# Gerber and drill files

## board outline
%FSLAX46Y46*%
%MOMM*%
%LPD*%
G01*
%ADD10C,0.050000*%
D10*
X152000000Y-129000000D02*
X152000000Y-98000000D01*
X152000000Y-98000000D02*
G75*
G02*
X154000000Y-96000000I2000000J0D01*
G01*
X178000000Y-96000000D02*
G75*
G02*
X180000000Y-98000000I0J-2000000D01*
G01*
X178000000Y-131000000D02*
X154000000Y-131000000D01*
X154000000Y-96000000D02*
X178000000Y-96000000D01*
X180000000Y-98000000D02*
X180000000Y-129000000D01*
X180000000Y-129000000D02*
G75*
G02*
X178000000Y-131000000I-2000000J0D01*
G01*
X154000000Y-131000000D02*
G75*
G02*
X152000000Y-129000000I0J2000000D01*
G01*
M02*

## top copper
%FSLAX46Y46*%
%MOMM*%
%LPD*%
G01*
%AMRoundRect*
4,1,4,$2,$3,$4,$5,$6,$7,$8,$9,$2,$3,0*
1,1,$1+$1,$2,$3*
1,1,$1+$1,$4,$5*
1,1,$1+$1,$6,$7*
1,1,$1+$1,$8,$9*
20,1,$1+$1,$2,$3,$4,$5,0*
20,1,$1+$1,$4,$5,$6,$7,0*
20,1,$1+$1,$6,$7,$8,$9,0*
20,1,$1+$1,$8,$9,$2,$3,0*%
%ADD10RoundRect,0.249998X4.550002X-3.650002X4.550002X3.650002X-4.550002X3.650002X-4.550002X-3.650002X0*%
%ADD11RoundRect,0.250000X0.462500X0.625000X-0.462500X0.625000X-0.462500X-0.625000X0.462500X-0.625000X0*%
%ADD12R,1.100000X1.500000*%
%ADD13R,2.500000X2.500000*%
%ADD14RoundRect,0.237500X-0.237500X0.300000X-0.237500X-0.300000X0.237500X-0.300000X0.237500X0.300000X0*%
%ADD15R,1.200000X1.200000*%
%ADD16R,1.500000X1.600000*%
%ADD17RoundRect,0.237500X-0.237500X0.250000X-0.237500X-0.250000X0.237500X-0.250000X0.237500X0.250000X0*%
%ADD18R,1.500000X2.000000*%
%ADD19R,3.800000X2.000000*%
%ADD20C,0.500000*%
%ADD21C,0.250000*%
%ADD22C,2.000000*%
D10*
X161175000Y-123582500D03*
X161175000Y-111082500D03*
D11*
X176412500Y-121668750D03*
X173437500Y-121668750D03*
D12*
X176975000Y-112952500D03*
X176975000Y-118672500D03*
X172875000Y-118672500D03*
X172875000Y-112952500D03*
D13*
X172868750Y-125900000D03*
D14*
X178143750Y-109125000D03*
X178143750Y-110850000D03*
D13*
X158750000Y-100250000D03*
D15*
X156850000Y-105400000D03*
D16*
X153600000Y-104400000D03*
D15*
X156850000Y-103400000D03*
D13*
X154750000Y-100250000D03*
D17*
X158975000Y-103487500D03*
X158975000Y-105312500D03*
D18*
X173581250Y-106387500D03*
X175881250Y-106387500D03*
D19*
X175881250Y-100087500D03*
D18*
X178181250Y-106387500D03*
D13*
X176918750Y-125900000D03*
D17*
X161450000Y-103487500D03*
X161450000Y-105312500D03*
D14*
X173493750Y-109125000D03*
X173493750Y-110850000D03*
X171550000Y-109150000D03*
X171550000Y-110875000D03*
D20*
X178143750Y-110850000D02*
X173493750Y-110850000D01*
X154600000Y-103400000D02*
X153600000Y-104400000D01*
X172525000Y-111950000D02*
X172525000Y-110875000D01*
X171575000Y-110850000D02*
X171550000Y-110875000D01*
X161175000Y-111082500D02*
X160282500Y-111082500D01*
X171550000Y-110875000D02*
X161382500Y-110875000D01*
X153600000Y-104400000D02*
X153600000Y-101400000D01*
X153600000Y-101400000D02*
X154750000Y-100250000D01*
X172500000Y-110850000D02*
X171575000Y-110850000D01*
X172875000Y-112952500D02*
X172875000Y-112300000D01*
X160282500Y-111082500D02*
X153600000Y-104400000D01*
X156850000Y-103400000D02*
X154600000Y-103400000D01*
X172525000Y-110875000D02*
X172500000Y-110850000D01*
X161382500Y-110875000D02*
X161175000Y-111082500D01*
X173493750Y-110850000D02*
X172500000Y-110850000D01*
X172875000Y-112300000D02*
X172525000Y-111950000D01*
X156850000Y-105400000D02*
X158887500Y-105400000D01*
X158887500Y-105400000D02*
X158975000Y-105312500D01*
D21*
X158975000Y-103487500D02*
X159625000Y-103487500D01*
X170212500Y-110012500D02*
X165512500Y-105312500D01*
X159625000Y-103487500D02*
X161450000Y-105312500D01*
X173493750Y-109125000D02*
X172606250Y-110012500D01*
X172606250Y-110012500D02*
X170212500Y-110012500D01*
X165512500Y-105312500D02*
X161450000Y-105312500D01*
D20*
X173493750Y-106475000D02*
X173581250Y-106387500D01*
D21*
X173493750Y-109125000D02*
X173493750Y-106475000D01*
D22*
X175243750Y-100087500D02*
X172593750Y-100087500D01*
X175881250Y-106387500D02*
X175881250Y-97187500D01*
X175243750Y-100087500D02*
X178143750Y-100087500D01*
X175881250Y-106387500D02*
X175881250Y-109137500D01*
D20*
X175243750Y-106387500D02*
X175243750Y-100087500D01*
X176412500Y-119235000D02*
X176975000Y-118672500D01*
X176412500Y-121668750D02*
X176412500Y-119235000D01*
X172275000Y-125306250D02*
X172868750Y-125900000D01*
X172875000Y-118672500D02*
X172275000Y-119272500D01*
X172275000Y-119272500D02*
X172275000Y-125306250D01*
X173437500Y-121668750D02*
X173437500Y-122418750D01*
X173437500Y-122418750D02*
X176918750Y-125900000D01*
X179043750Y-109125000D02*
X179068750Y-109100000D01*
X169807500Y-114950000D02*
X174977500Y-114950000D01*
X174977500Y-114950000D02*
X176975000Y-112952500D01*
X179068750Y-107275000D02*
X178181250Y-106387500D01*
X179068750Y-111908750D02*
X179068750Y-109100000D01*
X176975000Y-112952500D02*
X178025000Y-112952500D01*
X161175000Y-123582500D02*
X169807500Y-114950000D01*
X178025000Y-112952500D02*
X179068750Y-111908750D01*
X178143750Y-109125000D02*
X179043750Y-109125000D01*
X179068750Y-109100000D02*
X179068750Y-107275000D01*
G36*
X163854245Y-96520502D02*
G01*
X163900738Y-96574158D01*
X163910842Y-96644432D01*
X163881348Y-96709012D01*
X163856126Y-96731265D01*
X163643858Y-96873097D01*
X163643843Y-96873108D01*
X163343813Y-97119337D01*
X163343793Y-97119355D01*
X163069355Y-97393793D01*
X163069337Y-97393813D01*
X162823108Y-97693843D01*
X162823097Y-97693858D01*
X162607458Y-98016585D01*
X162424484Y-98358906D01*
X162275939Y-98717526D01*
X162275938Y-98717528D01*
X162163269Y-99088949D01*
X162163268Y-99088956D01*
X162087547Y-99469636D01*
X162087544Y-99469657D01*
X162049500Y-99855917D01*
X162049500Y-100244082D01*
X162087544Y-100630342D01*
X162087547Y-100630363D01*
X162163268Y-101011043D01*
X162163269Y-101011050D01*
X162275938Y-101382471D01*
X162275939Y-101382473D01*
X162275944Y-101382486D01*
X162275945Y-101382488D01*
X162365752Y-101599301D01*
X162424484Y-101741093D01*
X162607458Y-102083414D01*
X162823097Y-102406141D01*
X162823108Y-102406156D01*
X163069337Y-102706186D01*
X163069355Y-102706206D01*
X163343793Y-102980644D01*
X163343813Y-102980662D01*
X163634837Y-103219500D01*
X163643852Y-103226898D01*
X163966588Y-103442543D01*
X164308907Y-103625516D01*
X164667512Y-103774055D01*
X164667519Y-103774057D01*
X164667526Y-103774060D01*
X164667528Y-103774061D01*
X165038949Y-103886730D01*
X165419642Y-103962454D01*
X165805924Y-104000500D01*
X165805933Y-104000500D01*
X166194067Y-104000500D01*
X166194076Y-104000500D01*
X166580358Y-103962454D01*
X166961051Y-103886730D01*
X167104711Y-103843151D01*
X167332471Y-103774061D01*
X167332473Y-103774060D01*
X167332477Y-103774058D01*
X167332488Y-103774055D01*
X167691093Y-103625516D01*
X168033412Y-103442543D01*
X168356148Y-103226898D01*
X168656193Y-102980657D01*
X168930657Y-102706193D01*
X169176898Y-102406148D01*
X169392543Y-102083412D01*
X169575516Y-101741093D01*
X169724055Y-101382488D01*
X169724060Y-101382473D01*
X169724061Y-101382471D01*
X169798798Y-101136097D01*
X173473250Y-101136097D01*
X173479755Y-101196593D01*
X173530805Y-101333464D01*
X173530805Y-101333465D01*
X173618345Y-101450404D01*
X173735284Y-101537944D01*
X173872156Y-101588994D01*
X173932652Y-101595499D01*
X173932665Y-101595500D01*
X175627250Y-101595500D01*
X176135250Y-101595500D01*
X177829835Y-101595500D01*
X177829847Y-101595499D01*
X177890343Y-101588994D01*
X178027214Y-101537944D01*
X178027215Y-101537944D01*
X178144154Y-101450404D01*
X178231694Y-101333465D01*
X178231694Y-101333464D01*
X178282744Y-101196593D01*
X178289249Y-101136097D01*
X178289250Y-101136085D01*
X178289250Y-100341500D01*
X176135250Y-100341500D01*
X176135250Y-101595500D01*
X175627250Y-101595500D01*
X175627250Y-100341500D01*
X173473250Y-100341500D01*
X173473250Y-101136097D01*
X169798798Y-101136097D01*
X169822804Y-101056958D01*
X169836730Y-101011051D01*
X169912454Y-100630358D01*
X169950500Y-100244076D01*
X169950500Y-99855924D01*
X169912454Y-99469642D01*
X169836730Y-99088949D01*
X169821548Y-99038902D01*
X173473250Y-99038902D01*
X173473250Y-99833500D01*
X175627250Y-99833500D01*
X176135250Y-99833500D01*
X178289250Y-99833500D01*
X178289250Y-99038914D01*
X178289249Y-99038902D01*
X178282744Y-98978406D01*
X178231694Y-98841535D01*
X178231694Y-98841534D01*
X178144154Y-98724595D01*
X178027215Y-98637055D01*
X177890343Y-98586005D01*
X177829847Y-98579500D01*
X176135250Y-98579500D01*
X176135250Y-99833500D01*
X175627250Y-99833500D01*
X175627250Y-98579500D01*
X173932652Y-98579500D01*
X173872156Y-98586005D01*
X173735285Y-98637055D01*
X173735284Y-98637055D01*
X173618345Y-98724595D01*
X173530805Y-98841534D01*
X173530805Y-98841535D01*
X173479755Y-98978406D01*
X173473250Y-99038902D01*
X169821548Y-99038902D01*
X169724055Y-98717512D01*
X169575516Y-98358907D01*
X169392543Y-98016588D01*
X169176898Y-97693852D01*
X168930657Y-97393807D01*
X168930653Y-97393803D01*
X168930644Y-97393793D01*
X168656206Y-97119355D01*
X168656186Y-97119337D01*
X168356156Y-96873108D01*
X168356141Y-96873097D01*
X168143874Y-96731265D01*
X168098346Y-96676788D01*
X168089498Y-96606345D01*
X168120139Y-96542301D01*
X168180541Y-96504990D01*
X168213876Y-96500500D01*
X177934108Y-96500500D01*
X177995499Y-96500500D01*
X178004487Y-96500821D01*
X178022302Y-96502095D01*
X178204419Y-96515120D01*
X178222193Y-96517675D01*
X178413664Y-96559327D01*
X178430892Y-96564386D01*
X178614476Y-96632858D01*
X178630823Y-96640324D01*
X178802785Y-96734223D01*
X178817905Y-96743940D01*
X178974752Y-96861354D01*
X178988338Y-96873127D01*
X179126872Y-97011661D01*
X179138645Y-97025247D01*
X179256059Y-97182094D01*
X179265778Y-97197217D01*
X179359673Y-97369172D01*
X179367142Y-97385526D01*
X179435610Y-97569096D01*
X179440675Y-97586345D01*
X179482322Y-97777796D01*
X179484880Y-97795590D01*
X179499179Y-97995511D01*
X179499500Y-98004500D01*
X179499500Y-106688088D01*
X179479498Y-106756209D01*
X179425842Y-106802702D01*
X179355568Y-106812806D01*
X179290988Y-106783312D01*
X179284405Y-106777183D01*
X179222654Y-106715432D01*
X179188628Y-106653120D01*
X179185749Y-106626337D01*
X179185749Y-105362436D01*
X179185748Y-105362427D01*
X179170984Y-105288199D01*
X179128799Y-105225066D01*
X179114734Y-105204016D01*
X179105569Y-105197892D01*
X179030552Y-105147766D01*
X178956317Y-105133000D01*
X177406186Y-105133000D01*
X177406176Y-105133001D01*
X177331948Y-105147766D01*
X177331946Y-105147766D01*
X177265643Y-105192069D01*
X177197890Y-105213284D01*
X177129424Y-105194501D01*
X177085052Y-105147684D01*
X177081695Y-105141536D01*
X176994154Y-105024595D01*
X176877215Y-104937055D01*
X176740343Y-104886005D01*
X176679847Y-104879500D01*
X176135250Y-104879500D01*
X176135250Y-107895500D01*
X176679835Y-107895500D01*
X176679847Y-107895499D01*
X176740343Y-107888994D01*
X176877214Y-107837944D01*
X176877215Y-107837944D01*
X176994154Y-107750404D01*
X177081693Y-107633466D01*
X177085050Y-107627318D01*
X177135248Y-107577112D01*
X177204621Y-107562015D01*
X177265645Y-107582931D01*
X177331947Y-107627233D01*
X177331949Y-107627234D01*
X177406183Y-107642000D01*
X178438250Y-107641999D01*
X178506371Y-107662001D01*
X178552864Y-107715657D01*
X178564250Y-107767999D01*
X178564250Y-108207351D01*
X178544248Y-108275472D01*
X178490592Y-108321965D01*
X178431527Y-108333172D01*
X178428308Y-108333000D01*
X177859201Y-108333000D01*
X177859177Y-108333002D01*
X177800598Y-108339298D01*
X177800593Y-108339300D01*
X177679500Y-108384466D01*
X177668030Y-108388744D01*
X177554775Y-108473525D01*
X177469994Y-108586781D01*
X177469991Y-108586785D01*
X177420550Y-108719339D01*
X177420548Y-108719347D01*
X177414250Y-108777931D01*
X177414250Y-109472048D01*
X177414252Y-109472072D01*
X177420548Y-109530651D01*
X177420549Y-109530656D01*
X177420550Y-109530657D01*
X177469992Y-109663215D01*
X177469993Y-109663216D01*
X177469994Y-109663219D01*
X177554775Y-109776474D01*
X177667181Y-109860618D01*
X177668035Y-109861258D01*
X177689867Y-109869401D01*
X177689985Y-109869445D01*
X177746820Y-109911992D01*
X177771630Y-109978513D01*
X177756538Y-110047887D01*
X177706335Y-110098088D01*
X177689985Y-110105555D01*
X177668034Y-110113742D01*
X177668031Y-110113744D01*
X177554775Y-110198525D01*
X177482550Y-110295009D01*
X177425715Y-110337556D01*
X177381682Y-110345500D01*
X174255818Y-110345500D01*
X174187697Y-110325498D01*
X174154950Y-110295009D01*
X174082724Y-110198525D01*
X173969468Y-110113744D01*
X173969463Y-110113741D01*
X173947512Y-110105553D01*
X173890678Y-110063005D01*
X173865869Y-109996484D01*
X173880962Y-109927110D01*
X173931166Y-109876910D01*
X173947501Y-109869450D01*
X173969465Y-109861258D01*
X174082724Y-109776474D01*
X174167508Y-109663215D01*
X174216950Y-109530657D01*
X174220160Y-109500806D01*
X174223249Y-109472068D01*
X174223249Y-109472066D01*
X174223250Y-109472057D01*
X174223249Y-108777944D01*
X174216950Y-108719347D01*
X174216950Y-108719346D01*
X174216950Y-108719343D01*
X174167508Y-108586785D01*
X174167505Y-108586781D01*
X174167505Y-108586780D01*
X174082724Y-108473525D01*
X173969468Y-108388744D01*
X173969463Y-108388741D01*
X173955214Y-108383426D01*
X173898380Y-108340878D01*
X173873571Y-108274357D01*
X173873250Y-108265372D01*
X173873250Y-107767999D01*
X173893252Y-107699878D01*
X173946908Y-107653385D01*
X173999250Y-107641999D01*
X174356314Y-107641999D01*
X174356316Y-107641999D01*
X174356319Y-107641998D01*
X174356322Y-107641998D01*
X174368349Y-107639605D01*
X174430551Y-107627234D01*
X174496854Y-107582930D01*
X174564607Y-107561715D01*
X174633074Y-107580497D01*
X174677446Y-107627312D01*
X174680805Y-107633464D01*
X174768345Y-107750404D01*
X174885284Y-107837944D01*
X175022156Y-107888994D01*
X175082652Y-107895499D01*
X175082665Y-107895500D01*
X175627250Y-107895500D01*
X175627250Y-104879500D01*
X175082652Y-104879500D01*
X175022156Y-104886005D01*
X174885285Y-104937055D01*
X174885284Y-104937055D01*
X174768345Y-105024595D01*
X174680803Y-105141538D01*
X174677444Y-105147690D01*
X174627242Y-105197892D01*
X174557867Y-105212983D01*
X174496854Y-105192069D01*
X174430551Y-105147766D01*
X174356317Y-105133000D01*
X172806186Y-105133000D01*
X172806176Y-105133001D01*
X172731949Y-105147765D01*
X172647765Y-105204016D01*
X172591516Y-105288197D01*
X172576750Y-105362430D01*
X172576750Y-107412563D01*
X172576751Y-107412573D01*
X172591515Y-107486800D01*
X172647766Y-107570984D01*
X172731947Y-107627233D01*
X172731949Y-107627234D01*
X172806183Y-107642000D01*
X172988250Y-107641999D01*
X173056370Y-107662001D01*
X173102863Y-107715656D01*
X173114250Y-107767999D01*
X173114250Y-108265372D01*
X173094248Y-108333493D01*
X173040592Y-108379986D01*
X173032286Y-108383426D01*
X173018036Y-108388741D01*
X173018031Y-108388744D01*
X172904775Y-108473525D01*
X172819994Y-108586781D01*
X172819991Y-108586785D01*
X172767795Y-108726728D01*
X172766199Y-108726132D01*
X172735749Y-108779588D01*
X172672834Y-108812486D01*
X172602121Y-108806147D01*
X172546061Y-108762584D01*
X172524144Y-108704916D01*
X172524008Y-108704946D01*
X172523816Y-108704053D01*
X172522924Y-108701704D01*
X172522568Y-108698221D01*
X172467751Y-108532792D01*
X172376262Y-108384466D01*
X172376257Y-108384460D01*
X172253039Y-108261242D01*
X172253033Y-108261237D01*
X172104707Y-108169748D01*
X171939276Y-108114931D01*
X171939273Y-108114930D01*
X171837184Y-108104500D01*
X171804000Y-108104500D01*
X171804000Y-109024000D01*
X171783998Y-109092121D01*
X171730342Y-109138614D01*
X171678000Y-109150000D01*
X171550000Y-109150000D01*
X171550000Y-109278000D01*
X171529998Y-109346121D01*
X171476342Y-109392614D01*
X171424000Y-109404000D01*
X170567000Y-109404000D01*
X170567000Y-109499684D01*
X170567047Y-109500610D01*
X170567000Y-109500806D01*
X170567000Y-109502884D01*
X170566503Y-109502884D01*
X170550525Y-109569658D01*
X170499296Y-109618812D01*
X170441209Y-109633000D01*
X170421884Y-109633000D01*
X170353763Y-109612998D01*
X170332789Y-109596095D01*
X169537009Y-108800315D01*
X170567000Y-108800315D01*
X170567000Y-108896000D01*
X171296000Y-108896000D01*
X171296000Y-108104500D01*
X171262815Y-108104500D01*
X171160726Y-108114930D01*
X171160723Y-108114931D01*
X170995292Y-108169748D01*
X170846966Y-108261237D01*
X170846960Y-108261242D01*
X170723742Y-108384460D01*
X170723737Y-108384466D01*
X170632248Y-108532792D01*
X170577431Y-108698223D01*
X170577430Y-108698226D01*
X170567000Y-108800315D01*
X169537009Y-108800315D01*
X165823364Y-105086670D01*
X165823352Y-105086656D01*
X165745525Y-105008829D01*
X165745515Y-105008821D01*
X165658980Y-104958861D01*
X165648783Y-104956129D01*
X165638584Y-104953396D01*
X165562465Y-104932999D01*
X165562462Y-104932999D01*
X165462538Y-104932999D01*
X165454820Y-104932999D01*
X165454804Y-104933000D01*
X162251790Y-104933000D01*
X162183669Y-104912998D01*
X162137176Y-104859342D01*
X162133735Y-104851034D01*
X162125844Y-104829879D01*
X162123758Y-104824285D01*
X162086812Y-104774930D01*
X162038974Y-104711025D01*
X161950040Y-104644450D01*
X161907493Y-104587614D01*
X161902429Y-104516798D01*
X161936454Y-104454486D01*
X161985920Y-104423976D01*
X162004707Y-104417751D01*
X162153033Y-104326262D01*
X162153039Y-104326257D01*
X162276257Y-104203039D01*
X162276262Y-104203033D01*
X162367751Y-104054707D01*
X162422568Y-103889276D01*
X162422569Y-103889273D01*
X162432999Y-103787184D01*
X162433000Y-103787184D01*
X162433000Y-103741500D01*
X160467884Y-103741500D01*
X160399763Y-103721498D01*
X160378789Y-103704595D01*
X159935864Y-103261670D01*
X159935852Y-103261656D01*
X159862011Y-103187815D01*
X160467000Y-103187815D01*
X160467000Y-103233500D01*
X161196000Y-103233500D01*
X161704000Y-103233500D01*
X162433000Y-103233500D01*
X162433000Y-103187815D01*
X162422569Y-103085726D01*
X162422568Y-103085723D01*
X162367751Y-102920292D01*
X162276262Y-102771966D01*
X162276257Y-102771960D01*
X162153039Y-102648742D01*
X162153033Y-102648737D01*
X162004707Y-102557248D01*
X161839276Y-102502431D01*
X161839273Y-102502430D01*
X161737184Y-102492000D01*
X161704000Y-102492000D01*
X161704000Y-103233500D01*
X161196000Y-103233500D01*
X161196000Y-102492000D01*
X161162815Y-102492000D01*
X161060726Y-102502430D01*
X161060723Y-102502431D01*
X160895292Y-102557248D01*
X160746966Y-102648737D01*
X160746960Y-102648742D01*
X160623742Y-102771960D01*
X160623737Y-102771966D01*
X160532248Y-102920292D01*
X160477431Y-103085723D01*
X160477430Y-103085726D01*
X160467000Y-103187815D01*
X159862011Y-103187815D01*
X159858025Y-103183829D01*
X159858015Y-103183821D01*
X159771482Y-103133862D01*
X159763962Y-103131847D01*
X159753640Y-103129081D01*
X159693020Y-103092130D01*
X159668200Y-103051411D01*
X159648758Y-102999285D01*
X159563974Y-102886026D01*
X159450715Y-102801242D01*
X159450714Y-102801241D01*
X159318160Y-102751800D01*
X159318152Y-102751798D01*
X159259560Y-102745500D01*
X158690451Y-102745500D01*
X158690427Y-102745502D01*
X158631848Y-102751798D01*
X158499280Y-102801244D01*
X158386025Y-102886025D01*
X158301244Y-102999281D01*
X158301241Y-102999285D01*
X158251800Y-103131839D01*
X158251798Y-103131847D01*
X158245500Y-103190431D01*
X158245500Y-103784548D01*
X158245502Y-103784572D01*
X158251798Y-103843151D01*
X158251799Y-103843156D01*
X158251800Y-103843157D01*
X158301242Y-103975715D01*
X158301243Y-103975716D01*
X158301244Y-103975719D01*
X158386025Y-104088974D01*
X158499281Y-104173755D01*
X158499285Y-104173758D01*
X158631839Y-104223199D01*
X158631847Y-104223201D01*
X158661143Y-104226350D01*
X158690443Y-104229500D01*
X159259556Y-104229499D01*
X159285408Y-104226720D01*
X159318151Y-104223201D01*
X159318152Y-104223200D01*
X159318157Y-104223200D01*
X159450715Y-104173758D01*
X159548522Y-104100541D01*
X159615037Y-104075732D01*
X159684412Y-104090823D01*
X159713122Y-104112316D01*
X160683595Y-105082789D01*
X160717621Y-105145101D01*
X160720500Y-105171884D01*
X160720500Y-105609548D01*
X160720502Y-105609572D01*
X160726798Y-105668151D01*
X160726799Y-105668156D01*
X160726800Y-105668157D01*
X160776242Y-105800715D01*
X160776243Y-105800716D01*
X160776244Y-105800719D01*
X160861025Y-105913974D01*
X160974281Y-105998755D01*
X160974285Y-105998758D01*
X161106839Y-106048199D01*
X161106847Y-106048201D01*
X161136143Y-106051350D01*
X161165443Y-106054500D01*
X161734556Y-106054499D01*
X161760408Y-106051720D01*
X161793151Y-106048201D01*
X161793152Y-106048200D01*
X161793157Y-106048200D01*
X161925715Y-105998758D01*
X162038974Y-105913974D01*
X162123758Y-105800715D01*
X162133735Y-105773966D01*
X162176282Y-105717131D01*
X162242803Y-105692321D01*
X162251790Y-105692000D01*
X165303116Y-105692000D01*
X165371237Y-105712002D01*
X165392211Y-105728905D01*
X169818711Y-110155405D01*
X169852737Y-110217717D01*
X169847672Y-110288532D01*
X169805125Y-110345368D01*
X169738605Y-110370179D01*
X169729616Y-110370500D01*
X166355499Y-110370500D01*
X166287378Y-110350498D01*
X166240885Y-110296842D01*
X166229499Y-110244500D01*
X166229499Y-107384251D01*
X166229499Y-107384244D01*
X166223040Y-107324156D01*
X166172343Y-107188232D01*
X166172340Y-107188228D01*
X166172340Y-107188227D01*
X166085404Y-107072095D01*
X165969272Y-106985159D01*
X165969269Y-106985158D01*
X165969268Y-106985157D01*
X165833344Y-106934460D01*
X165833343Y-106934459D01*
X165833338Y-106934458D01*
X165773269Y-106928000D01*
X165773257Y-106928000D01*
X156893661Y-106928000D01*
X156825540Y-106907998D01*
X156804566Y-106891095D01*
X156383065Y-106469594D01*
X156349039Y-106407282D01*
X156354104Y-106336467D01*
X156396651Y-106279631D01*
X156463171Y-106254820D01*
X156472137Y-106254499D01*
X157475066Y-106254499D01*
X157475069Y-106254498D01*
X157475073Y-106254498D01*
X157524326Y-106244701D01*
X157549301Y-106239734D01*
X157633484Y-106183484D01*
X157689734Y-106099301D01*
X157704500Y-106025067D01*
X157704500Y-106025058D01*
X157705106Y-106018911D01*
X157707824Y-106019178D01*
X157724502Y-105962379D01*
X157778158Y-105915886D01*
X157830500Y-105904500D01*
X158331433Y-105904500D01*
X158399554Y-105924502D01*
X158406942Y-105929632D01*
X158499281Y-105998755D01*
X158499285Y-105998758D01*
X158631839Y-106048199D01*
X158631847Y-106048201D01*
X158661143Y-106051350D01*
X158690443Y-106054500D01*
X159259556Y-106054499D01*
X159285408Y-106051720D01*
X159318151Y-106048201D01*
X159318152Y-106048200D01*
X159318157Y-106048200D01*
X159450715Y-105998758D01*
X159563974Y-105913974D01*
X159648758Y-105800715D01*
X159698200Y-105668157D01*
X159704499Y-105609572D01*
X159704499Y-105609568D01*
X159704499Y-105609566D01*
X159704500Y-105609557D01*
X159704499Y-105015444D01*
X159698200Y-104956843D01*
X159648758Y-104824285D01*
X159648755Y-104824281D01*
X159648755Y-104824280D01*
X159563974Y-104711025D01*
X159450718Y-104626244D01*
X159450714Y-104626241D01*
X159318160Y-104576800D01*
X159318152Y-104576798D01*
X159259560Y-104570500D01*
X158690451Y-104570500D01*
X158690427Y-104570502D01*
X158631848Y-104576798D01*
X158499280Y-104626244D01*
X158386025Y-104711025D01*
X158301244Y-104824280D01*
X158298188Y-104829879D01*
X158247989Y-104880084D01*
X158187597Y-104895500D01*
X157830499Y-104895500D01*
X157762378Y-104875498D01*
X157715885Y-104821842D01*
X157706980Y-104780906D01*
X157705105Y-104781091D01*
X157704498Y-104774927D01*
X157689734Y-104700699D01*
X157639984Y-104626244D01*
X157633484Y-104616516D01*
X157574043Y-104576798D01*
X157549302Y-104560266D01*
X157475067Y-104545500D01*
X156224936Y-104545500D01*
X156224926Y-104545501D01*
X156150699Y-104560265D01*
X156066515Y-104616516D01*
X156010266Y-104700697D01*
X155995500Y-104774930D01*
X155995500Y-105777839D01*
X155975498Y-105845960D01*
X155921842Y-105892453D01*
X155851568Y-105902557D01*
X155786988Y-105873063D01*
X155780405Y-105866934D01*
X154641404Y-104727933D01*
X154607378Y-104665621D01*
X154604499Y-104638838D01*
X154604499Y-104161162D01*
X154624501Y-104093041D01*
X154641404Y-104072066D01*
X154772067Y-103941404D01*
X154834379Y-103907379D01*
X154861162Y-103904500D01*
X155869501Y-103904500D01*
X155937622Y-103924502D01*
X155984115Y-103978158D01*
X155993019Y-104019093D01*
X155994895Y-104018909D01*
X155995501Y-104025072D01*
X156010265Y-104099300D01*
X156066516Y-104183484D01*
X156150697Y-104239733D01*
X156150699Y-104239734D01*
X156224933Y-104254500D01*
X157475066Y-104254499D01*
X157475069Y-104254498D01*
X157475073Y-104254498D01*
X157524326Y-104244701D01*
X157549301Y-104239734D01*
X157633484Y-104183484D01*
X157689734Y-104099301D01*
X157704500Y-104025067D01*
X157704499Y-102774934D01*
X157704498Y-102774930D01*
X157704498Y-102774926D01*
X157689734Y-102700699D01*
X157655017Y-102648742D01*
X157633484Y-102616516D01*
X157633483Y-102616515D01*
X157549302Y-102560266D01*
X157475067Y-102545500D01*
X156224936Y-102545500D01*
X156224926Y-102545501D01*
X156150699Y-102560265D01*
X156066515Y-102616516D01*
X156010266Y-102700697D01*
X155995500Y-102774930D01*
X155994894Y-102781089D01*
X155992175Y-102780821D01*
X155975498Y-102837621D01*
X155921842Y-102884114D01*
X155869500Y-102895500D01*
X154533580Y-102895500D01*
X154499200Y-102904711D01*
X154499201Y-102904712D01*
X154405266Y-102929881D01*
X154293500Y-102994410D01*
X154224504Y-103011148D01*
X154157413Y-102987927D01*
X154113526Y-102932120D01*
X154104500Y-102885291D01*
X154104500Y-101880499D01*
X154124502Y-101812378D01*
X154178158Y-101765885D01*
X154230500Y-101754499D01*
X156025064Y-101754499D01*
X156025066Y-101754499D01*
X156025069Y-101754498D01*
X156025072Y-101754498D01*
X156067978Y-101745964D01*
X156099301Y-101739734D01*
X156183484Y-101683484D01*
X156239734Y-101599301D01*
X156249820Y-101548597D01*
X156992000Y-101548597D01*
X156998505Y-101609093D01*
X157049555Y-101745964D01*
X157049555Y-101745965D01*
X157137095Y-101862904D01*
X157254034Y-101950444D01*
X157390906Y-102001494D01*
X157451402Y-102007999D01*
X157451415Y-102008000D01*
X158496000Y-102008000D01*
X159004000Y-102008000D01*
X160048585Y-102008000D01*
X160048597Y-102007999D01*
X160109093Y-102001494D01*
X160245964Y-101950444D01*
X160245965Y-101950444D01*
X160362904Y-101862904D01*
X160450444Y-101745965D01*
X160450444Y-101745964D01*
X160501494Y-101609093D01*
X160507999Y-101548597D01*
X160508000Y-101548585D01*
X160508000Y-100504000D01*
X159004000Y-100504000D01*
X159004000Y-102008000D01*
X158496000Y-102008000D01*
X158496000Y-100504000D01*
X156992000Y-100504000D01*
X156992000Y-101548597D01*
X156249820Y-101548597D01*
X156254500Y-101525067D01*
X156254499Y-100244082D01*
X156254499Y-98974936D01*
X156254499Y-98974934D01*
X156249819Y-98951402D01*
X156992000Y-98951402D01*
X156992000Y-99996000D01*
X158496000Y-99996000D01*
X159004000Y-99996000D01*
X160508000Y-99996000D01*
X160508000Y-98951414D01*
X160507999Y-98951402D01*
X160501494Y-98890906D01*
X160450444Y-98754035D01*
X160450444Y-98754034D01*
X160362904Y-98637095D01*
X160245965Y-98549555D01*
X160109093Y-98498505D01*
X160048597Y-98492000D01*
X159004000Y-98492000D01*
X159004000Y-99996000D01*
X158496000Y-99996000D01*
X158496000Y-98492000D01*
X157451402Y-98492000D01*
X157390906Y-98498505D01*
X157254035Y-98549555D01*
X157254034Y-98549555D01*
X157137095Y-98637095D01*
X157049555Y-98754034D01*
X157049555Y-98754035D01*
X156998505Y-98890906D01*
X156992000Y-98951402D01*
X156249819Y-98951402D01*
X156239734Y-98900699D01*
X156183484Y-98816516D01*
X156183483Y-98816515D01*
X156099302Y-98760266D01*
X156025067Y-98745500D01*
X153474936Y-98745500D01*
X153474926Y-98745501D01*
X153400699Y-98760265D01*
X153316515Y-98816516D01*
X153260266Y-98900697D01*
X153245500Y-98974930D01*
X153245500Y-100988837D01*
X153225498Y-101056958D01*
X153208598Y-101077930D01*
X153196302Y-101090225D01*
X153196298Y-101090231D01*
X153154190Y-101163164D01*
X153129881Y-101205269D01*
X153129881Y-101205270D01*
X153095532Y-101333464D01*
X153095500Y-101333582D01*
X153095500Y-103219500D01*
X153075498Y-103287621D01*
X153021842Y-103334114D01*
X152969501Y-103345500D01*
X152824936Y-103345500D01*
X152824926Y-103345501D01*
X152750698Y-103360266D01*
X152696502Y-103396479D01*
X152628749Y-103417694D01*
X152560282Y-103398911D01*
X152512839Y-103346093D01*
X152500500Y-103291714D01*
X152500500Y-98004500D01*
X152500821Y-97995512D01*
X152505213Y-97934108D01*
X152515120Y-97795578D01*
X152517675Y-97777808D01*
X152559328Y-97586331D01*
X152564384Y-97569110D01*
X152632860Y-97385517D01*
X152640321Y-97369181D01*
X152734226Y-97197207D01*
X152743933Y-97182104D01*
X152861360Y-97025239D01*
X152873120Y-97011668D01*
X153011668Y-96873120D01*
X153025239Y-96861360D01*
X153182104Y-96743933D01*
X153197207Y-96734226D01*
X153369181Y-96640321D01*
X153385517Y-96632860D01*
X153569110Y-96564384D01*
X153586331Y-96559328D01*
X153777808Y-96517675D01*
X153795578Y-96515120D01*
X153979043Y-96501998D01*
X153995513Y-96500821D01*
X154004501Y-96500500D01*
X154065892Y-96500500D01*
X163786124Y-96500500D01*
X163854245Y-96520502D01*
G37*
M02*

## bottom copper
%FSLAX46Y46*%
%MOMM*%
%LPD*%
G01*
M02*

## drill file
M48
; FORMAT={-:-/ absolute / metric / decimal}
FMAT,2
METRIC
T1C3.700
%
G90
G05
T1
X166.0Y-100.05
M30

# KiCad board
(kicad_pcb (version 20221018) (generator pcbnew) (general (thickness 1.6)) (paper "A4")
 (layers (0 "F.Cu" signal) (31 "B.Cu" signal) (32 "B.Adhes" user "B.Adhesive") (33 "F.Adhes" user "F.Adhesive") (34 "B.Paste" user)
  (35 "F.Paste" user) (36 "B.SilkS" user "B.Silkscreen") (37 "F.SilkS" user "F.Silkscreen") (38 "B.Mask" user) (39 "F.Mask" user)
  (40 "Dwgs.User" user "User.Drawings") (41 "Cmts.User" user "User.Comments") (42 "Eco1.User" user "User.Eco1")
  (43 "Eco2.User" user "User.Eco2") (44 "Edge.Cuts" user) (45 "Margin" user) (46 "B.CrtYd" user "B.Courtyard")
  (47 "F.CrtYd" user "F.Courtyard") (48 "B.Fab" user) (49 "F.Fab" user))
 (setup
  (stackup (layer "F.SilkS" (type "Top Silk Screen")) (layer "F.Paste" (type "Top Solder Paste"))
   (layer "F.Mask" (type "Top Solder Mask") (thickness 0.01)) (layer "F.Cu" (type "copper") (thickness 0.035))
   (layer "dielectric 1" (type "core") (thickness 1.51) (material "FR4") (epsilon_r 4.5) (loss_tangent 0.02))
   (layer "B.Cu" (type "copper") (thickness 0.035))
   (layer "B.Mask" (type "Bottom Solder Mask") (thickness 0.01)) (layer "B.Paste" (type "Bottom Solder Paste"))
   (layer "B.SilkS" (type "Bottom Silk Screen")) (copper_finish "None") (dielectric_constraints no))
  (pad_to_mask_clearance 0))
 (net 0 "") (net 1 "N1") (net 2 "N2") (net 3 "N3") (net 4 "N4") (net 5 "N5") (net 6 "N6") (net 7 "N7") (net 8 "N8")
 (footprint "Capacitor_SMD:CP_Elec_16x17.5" (layer "F.Cu") (at 161.175 117.3325 90)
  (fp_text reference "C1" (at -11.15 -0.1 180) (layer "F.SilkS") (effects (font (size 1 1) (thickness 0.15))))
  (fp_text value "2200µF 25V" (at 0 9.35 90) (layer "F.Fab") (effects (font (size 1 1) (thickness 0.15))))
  (pad "1" smd roundrect (at -6.25 0 90) (size 7.8 9.6) (layers "F.Cu" "F.Paste" "F.Mask") (roundrect_rratio 0.032051) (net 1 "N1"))
  (pad "2" smd roundrect (at 6.25 0 90) (size 7.8 9.6) (layers "F.Cu" "F.Paste" "F.Mask") (roundrect_rratio 0.032051) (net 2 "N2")))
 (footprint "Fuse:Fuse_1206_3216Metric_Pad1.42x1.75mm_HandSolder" (layer "F.Cu") (at 174.925 121.66875 180)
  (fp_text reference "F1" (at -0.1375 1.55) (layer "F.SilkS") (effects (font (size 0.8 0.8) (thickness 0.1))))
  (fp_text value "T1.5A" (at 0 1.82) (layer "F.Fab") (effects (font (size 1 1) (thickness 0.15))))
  (pad "1" smd roundrect (at -1.4875 0 180) (size 1.425 1.75) (layers "F.Cu" "F.Paste" "F.Mask") (roundrect_rratio 0.1754385965)
   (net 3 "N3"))
  (pad "2" smd roundrect (at 1.4875 0 180) (size 1.425 1.75) (layers "F.Cu" "F.Paste" "F.Mask") (roundrect_rratio 0.1754385965) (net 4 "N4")))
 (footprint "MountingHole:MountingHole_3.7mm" (layer "F.Cu") (at 166 100.05) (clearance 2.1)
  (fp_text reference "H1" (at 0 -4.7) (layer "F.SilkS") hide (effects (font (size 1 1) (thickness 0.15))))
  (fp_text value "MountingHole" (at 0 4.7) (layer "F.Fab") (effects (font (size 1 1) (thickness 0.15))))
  (pad "" np_thru_hole circle (at 0 0) (size 3.7 3.7) (drill 3.7) (layers "*.Cu" "*.Mask")))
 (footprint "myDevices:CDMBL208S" (layer "F.Cu") (at 174.925 115.8125)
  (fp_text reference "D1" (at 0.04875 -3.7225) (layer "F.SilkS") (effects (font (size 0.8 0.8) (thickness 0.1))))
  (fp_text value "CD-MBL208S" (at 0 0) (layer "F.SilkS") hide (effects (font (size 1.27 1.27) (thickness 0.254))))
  (pad "1" smd rect (at 2.05 -2.86) (size 1.1 1.5) (layers "F.Cu" "F.Paste" "F.Mask") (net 1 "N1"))
  (pad "2" smd rect (at 2.05 2.86) (size 1.1 1.5) (layers "F.Cu" "F.Paste" "F.Mask") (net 3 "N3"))
  (pad "3" smd rect (at -2.05 2.86) (size 1.1 1.5) (layers "F.Cu" "F.Paste" "F.Mask") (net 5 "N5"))
  (pad "4" smd rect (at -2.05 -2.86) (size 1.1 1.5) (layers "F.Cu" "F.Paste" "F.Mask") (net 2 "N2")))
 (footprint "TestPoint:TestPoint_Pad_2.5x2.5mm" (layer "F.Cu") (at 172.86875 125.9)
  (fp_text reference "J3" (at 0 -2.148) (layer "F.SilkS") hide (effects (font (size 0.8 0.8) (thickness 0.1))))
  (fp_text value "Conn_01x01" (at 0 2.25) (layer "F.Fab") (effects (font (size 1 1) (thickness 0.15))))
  (pad "1" smd rect (at 0 0) (size 2.5 2.5) (layers "F.Cu" "F.Mask") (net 5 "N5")))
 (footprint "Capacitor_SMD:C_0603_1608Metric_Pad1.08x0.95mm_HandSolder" (layer "F.Cu") (at 178.14375 109.9875 -90)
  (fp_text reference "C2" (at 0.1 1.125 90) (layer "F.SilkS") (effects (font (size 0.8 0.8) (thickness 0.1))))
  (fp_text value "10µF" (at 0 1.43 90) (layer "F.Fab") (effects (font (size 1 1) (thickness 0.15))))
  (pad "1" smd roundrect (at -0.8625 0 270) (size 1.075 0.95) (layers "F.Cu" "F.Paste" "F.Mask") (roundrect_rratio 0.25) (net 1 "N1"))
  (pad "2" smd roundrect (at 0.8625 0 270) (size 1.075 0.95) (layers "F.Cu" "F.Paste" "F.Mask") (roundrect_rratio 0.25) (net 2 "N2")))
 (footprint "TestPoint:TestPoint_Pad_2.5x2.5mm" (layer "F.Cu") (at 158.75 100.25)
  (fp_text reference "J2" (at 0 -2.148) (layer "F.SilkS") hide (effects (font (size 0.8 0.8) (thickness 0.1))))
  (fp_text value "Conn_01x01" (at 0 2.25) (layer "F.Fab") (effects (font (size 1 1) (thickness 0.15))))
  (pad "1" smd rect (at 0 0) (size 2.5 2.5) (layers "F.Cu" "F.Mask") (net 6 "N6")))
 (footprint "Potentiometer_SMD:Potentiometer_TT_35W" (layer "F.Cu") (at 155.05 104.4 180)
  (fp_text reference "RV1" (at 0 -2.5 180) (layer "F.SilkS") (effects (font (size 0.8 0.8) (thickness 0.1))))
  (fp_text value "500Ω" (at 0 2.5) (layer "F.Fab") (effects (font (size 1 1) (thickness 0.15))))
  (pad "1" smd rect (at -1.8 -1 180) (size 1.2 1.2) (layers "F.Cu" "F.Paste" "F.Mask") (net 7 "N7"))
  (pad "2" smd rect (at 1.45 0 180) (size 1.5 1.6) (layers "F.Cu" "F.Paste" "F.Mask") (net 2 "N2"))
  (pad "3" smd rect (at -1.8 1 180) (size 1.2 1.2) (layers "F.Cu" "F.Paste" "F.Mask") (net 2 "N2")))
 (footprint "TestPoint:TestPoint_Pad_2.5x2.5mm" (layer "F.Cu") (at 154.75 100.25)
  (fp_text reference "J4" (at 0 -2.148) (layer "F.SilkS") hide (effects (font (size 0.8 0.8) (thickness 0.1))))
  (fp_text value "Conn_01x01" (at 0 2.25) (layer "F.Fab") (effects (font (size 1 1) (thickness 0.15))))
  (pad "1" smd rect (at 0 0) (size 2.5 2.5) (layers "F.Cu" "F.Mask") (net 2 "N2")))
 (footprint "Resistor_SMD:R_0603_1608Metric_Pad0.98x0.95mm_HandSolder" (layer "F.Cu") (at 158.975 104.4 -90)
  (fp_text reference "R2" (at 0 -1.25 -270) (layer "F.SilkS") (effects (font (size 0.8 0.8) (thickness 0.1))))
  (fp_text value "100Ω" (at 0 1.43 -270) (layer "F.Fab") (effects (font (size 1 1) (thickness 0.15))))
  (pad "1" smd roundrect (at -0.9125 0 270) (size 0.975 0.95) (layers "F.Cu" "F.Paste" "F.Mask") (roundrect_rratio 0.25) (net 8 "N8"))
  (pad "2" smd roundrect (at 0.9125 0 270) (size 0.975 0.95) (layers "F.Cu" "F.Paste" "F.Mask") (roundrect_rratio 0.25) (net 7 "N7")))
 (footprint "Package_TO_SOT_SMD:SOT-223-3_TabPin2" (layer "F.Cu") (at 175.88125 103.2375 90)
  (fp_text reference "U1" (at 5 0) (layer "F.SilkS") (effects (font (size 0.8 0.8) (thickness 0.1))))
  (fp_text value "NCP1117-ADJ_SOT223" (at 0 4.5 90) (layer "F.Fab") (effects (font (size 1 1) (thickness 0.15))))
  (pad "1" smd rect (at -3.15 -2.3 90) (size 2 1.5) (layers "F.Cu" "F.Paste" "F.Mask") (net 8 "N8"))
  (pad "2" smd rect (at -3.15 0 90) (size 2 1.5) (layers "F.Cu" "F.Paste" "F.Mask") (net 6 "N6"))
  (pad "2" smd rect (at 3.15 0 90) (size 2 3.8) (layers "F.Cu" "F.Paste" "F.Mask") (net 6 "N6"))
  (pad "3" smd rect (at -3.15 2.3 90) (size 2 1.5) (layers "F.Cu" "F.Paste" "F.Mask") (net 1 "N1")))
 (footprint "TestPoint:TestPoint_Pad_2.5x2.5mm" (layer "F.Cu") (at 176.91875 125.9)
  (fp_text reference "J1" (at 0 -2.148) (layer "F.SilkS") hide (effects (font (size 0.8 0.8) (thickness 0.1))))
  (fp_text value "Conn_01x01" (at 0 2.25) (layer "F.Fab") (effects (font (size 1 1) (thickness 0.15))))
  (pad "1" smd rect (at 0 0) (size 2.5 2.5) (layers "F.Cu" "F.Mask") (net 4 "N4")))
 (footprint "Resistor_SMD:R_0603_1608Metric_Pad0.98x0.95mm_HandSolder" (layer "F.Cu") (at 161.45 104.4 -90)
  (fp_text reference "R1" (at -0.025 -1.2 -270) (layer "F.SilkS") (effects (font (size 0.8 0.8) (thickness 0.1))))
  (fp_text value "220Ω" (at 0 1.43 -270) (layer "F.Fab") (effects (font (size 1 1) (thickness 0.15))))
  (pad "1" smd roundrect (at -0.9125 0 270) (size 0.975 0.95) (layers "F.Cu" "F.Paste" "F.Mask") (roundrect_rratio 0.25) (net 6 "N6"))
  (pad "2" smd roundrect (at 0.9125 0 270) (size 0.975 0.95) (layers "F.Cu" "F.Paste" "F.Mask") (roundrect_rratio 0.25) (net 8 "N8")))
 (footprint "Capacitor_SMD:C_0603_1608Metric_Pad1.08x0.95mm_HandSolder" (layer "F.Cu") (at 173.49375 109.9875 -90)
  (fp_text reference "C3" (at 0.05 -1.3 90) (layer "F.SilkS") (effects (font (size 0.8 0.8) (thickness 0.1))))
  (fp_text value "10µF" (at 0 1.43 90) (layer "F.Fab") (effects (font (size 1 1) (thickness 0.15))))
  (pad "1" smd roundrect (at -0.8625 0 270) (size 1.075 0.95) (layers "F.Cu" "F.Paste" "F.Mask") (roundrect_rratio 0.25) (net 8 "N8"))
  (pad "2" smd roundrect (at 0.8625 0 270) (size 1.075 0.95) (layers "F.Cu" "F.Paste" "F.Mask") (roundrect_rratio 0.25) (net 2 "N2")))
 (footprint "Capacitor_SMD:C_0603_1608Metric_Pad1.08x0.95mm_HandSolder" (layer "F.Cu") (at 171.55 110.0125 -90)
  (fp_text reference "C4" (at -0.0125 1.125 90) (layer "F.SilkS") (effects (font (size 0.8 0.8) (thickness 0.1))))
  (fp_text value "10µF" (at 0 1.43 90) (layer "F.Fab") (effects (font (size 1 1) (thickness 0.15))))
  (pad "1" smd roundrect (at -0.8625 0 270) (size 1.075 0.95) (layers "F.Cu" "F.Paste" "F.Mask") (roundrect_rratio 0.25) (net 6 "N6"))
  (pad "2" smd roundrect (at 0.8625 0 270) (size 1.075 0.95) (layers "F.Cu" "F.Paste" "F.Mask") (roundrect_rratio 0.25) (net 2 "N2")))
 (gr_line (start 152 129) (end 152 98) (stroke (width 0.05) (type solid)) (layer "Edge.Cuts"))
 (gr_arc (start 152 98) (mid 152.585786 96.585786) (end 154 96) (stroke (width 0.05) (type solid)) (layer "Edge.Cuts"))
 (gr_arc (start 178 96) (mid 179.414214 96.585786) (end 180 98) (stroke (width 0.05) (type solid)) (layer "Edge.Cuts"))
 (gr_line (start 178 131) (end 154 131) (stroke (width 0.05) (type solid)) (layer "Edge.Cuts"))
 (gr_line (start 154 96) (end 178 96) (stroke (width 0.05) (type solid)) (layer "Edge.Cuts"))
 (gr_line (start 180 98) (end 180 129) (stroke (width 0.05) (type solid)) (layer "Edge.Cuts"))
 (gr_arc (start 180 129) (mid 179.414214 130.414214) (end 178 131) (stroke (width 0.05) (type solid)) (layer "Edge.Cuts"))
 (gr_arc (start 154 131) (mid 152.585786 130.414214) (end 152 129) (stroke (width 0.05) (type solid)) (layer "Edge.Cuts"))
 (segment (start 178.14375 110.85) (end 173.49375 110.85) (width 0.5) (layer "F.Cu") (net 2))
 (segment (start 154.6 103.4) (end 153.6 104.4) (width 0.5) (layer "F.Cu") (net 2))
 (segment (start 172.525 111.95) (end 172.525 110.875) (width 0.5) (layer "F.Cu") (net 2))
 (segment (start 171.575 110.85) (end 171.55 110.875) (width 0.5) (layer "F.Cu") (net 2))
 (segment (start 161.175 111.0825) (end 160.2825 111.0825) (width 0.5) (layer "F.Cu") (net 2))
 (segment (start 171.55 110.875) (end 161.3825 110.875) (width 0.5) (layer "F.Cu") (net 2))
 (segment (start 153.6 104.4) (end 153.6 101.4) (width 0.5) (layer "F.Cu") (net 2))
 (segment (start 153.6 101.4) (end 154.75 100.25) (width 0.5) (layer "F.Cu") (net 2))
 (segment (start 172.5 110.85) (end 171.575 110.85) (width 0.5) (layer "F.Cu") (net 2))
 (segment (start 172.875 112.9525) (end 172.875 112.3) (width 0.5) (layer "F.Cu") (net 2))
 (segment (start 160.2825 111.0825) (end 153.6 104.4) (width 0.5) (layer "F.Cu") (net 2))
 (segment (start 156.85 103.4) (end 154.6 103.4) (width 0.5) (layer "F.Cu") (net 2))
 (segment (start 172.525 110.875) (end 172.5 110.85) (width 0.5) (layer "F.Cu") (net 2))
 (segment (start 161.3825 110.875) (end 161.175 111.0825) (width 0.5) (layer "F.Cu") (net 2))
 (segment (start 173.49375 110.85) (end 172.5 110.85) (width 0.5) (layer "F.Cu") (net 2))
 (segment (start 172.875 112.3) (end 172.525 111.95) (width 0.5) (layer "F.Cu") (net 2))
 (segment (start 156.85 105.4) (end 158.8875 105.4) (width 0.5) (layer "F.Cu") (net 7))
 (segment (start 158.8875 105.4) (end 158.975 105.3125) (width 0.5) (layer "F.Cu") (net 7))
 (segment (start 158.975 103.4875) (end 159.625 103.4875) (width 0.25) (layer "F.Cu") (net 8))
 (segment (start 170.2125 110.0125) (end 165.5125 105.3125) (width 0.25) (layer "F.Cu") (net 8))
 (segment (start 159.625 103.4875) (end 161.45 105.3125) (width 0.25) (layer "F.Cu") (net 8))
 (segment (start 173.49375 109.125) (end 172.60625 110.0125) (width 0.25) (layer "F.Cu") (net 8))
 (segment (start 172.60625 110.0125) (end 170.2125 110.0125) (width 0.25) (layer "F.Cu") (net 8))
 (segment (start 165.5125 105.3125) (end 161.45 105.3125) (width 0.25) (layer "F.Cu") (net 8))
 (segment (start 173.49375 106.475) (end 173.58125 106.3875) (width 0.5) (layer "F.Cu") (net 8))
 (segment (start 173.49375 109.125) (end 173.49375 106.475) (width 0.25) (layer "F.Cu") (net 8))
 (segment (start 175.24375 100.0875) (end 172.59375 100.0875) (width 2) (layer "F.Cu") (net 6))
 (segment (start 175.88125 106.3875) (end 175.88125 97.1875) (width 2) (layer "F.Cu") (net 6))
 (segment (start 175.24375 100.0875) (end 178.14375 100.0875) (width 2) (layer "F.Cu") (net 6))
 (segment (start 175.88125 106.3875) (end 175.88125 109.1375) (width 2) (layer "F.Cu") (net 6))
 (segment (start 175.24375 106.3875) (end 175.24375 100.0875) (width 0.5) (layer "F.Cu") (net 6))
 (segment (start 176.4125 119.235) (end 176.975 118.6725) (width 0.5) (layer "F.Cu") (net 3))
 (segment (start 176.4125 121.66875) (end 176.4125 119.235) (width 0.5) (layer "F.Cu") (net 3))
 (segment (start 172.275 125.30625) (end 172.86875 125.9) (width 0.5) (layer "F.Cu") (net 5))
 (segment (start 172.875 118.6725) (end 172.275 119.2725) (width 0.5) (layer "F.Cu") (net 5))
 (segment (start 172.275 119.2725) (end 172.275 125.30625) (width 0.5) (layer "F.Cu") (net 5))
 (segment (start 173.4375 121.66875) (end 173.4375 122.41875) (width 0.5) (layer "F.Cu") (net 4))
 (segment (start 173.4375 122.41875) (end 176.91875 125.9) (width 0.5) (layer "F.Cu") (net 4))
 (segment (start 179.04375 109.125) (end 179.06875 109.1) (width 0.5) (layer "F.Cu") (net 1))
 (segment (start 169.8075 114.95) (end 174.9775 114.95) (width 0.5) (layer "F.Cu") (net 1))
 (segment (start 174.9775 114.95) (end 176.975 112.9525) (width 0.5) (layer "F.Cu") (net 1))
 (segment (start 179.06875 107.275) (end 178.18125 106.3875) (width 0.5) (layer "F.Cu") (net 1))
 (segment (start 179.06875 111.90875) (end 179.06875 109.1) (width 0.5) (layer "F.Cu") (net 1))
 (segment (start 176.975 112.9525) (end 178.025 112.9525) (width 0.5) (layer "F.Cu") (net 1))
 (segment (start 161.175 123.5825) (end 169.8075 114.95) (width 0.5) (layer "F.Cu") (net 1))
 (segment (start 178.025 112.9525) (end 179.06875 111.90875) (width 0.5) (layer "F.Cu") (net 1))
 (segment (start 178.14375 109.125) (end 179.04375 109.125) (width 0.5) (layer "F.Cu") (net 1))
 (segment (start 179.06875 109.1) (end 179.06875 107.275) (width 0.5) (layer "F.Cu") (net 1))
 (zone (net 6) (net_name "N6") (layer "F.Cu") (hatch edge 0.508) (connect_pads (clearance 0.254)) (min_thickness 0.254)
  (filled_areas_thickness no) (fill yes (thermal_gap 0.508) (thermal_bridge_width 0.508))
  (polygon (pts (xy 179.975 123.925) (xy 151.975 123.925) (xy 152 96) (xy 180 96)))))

